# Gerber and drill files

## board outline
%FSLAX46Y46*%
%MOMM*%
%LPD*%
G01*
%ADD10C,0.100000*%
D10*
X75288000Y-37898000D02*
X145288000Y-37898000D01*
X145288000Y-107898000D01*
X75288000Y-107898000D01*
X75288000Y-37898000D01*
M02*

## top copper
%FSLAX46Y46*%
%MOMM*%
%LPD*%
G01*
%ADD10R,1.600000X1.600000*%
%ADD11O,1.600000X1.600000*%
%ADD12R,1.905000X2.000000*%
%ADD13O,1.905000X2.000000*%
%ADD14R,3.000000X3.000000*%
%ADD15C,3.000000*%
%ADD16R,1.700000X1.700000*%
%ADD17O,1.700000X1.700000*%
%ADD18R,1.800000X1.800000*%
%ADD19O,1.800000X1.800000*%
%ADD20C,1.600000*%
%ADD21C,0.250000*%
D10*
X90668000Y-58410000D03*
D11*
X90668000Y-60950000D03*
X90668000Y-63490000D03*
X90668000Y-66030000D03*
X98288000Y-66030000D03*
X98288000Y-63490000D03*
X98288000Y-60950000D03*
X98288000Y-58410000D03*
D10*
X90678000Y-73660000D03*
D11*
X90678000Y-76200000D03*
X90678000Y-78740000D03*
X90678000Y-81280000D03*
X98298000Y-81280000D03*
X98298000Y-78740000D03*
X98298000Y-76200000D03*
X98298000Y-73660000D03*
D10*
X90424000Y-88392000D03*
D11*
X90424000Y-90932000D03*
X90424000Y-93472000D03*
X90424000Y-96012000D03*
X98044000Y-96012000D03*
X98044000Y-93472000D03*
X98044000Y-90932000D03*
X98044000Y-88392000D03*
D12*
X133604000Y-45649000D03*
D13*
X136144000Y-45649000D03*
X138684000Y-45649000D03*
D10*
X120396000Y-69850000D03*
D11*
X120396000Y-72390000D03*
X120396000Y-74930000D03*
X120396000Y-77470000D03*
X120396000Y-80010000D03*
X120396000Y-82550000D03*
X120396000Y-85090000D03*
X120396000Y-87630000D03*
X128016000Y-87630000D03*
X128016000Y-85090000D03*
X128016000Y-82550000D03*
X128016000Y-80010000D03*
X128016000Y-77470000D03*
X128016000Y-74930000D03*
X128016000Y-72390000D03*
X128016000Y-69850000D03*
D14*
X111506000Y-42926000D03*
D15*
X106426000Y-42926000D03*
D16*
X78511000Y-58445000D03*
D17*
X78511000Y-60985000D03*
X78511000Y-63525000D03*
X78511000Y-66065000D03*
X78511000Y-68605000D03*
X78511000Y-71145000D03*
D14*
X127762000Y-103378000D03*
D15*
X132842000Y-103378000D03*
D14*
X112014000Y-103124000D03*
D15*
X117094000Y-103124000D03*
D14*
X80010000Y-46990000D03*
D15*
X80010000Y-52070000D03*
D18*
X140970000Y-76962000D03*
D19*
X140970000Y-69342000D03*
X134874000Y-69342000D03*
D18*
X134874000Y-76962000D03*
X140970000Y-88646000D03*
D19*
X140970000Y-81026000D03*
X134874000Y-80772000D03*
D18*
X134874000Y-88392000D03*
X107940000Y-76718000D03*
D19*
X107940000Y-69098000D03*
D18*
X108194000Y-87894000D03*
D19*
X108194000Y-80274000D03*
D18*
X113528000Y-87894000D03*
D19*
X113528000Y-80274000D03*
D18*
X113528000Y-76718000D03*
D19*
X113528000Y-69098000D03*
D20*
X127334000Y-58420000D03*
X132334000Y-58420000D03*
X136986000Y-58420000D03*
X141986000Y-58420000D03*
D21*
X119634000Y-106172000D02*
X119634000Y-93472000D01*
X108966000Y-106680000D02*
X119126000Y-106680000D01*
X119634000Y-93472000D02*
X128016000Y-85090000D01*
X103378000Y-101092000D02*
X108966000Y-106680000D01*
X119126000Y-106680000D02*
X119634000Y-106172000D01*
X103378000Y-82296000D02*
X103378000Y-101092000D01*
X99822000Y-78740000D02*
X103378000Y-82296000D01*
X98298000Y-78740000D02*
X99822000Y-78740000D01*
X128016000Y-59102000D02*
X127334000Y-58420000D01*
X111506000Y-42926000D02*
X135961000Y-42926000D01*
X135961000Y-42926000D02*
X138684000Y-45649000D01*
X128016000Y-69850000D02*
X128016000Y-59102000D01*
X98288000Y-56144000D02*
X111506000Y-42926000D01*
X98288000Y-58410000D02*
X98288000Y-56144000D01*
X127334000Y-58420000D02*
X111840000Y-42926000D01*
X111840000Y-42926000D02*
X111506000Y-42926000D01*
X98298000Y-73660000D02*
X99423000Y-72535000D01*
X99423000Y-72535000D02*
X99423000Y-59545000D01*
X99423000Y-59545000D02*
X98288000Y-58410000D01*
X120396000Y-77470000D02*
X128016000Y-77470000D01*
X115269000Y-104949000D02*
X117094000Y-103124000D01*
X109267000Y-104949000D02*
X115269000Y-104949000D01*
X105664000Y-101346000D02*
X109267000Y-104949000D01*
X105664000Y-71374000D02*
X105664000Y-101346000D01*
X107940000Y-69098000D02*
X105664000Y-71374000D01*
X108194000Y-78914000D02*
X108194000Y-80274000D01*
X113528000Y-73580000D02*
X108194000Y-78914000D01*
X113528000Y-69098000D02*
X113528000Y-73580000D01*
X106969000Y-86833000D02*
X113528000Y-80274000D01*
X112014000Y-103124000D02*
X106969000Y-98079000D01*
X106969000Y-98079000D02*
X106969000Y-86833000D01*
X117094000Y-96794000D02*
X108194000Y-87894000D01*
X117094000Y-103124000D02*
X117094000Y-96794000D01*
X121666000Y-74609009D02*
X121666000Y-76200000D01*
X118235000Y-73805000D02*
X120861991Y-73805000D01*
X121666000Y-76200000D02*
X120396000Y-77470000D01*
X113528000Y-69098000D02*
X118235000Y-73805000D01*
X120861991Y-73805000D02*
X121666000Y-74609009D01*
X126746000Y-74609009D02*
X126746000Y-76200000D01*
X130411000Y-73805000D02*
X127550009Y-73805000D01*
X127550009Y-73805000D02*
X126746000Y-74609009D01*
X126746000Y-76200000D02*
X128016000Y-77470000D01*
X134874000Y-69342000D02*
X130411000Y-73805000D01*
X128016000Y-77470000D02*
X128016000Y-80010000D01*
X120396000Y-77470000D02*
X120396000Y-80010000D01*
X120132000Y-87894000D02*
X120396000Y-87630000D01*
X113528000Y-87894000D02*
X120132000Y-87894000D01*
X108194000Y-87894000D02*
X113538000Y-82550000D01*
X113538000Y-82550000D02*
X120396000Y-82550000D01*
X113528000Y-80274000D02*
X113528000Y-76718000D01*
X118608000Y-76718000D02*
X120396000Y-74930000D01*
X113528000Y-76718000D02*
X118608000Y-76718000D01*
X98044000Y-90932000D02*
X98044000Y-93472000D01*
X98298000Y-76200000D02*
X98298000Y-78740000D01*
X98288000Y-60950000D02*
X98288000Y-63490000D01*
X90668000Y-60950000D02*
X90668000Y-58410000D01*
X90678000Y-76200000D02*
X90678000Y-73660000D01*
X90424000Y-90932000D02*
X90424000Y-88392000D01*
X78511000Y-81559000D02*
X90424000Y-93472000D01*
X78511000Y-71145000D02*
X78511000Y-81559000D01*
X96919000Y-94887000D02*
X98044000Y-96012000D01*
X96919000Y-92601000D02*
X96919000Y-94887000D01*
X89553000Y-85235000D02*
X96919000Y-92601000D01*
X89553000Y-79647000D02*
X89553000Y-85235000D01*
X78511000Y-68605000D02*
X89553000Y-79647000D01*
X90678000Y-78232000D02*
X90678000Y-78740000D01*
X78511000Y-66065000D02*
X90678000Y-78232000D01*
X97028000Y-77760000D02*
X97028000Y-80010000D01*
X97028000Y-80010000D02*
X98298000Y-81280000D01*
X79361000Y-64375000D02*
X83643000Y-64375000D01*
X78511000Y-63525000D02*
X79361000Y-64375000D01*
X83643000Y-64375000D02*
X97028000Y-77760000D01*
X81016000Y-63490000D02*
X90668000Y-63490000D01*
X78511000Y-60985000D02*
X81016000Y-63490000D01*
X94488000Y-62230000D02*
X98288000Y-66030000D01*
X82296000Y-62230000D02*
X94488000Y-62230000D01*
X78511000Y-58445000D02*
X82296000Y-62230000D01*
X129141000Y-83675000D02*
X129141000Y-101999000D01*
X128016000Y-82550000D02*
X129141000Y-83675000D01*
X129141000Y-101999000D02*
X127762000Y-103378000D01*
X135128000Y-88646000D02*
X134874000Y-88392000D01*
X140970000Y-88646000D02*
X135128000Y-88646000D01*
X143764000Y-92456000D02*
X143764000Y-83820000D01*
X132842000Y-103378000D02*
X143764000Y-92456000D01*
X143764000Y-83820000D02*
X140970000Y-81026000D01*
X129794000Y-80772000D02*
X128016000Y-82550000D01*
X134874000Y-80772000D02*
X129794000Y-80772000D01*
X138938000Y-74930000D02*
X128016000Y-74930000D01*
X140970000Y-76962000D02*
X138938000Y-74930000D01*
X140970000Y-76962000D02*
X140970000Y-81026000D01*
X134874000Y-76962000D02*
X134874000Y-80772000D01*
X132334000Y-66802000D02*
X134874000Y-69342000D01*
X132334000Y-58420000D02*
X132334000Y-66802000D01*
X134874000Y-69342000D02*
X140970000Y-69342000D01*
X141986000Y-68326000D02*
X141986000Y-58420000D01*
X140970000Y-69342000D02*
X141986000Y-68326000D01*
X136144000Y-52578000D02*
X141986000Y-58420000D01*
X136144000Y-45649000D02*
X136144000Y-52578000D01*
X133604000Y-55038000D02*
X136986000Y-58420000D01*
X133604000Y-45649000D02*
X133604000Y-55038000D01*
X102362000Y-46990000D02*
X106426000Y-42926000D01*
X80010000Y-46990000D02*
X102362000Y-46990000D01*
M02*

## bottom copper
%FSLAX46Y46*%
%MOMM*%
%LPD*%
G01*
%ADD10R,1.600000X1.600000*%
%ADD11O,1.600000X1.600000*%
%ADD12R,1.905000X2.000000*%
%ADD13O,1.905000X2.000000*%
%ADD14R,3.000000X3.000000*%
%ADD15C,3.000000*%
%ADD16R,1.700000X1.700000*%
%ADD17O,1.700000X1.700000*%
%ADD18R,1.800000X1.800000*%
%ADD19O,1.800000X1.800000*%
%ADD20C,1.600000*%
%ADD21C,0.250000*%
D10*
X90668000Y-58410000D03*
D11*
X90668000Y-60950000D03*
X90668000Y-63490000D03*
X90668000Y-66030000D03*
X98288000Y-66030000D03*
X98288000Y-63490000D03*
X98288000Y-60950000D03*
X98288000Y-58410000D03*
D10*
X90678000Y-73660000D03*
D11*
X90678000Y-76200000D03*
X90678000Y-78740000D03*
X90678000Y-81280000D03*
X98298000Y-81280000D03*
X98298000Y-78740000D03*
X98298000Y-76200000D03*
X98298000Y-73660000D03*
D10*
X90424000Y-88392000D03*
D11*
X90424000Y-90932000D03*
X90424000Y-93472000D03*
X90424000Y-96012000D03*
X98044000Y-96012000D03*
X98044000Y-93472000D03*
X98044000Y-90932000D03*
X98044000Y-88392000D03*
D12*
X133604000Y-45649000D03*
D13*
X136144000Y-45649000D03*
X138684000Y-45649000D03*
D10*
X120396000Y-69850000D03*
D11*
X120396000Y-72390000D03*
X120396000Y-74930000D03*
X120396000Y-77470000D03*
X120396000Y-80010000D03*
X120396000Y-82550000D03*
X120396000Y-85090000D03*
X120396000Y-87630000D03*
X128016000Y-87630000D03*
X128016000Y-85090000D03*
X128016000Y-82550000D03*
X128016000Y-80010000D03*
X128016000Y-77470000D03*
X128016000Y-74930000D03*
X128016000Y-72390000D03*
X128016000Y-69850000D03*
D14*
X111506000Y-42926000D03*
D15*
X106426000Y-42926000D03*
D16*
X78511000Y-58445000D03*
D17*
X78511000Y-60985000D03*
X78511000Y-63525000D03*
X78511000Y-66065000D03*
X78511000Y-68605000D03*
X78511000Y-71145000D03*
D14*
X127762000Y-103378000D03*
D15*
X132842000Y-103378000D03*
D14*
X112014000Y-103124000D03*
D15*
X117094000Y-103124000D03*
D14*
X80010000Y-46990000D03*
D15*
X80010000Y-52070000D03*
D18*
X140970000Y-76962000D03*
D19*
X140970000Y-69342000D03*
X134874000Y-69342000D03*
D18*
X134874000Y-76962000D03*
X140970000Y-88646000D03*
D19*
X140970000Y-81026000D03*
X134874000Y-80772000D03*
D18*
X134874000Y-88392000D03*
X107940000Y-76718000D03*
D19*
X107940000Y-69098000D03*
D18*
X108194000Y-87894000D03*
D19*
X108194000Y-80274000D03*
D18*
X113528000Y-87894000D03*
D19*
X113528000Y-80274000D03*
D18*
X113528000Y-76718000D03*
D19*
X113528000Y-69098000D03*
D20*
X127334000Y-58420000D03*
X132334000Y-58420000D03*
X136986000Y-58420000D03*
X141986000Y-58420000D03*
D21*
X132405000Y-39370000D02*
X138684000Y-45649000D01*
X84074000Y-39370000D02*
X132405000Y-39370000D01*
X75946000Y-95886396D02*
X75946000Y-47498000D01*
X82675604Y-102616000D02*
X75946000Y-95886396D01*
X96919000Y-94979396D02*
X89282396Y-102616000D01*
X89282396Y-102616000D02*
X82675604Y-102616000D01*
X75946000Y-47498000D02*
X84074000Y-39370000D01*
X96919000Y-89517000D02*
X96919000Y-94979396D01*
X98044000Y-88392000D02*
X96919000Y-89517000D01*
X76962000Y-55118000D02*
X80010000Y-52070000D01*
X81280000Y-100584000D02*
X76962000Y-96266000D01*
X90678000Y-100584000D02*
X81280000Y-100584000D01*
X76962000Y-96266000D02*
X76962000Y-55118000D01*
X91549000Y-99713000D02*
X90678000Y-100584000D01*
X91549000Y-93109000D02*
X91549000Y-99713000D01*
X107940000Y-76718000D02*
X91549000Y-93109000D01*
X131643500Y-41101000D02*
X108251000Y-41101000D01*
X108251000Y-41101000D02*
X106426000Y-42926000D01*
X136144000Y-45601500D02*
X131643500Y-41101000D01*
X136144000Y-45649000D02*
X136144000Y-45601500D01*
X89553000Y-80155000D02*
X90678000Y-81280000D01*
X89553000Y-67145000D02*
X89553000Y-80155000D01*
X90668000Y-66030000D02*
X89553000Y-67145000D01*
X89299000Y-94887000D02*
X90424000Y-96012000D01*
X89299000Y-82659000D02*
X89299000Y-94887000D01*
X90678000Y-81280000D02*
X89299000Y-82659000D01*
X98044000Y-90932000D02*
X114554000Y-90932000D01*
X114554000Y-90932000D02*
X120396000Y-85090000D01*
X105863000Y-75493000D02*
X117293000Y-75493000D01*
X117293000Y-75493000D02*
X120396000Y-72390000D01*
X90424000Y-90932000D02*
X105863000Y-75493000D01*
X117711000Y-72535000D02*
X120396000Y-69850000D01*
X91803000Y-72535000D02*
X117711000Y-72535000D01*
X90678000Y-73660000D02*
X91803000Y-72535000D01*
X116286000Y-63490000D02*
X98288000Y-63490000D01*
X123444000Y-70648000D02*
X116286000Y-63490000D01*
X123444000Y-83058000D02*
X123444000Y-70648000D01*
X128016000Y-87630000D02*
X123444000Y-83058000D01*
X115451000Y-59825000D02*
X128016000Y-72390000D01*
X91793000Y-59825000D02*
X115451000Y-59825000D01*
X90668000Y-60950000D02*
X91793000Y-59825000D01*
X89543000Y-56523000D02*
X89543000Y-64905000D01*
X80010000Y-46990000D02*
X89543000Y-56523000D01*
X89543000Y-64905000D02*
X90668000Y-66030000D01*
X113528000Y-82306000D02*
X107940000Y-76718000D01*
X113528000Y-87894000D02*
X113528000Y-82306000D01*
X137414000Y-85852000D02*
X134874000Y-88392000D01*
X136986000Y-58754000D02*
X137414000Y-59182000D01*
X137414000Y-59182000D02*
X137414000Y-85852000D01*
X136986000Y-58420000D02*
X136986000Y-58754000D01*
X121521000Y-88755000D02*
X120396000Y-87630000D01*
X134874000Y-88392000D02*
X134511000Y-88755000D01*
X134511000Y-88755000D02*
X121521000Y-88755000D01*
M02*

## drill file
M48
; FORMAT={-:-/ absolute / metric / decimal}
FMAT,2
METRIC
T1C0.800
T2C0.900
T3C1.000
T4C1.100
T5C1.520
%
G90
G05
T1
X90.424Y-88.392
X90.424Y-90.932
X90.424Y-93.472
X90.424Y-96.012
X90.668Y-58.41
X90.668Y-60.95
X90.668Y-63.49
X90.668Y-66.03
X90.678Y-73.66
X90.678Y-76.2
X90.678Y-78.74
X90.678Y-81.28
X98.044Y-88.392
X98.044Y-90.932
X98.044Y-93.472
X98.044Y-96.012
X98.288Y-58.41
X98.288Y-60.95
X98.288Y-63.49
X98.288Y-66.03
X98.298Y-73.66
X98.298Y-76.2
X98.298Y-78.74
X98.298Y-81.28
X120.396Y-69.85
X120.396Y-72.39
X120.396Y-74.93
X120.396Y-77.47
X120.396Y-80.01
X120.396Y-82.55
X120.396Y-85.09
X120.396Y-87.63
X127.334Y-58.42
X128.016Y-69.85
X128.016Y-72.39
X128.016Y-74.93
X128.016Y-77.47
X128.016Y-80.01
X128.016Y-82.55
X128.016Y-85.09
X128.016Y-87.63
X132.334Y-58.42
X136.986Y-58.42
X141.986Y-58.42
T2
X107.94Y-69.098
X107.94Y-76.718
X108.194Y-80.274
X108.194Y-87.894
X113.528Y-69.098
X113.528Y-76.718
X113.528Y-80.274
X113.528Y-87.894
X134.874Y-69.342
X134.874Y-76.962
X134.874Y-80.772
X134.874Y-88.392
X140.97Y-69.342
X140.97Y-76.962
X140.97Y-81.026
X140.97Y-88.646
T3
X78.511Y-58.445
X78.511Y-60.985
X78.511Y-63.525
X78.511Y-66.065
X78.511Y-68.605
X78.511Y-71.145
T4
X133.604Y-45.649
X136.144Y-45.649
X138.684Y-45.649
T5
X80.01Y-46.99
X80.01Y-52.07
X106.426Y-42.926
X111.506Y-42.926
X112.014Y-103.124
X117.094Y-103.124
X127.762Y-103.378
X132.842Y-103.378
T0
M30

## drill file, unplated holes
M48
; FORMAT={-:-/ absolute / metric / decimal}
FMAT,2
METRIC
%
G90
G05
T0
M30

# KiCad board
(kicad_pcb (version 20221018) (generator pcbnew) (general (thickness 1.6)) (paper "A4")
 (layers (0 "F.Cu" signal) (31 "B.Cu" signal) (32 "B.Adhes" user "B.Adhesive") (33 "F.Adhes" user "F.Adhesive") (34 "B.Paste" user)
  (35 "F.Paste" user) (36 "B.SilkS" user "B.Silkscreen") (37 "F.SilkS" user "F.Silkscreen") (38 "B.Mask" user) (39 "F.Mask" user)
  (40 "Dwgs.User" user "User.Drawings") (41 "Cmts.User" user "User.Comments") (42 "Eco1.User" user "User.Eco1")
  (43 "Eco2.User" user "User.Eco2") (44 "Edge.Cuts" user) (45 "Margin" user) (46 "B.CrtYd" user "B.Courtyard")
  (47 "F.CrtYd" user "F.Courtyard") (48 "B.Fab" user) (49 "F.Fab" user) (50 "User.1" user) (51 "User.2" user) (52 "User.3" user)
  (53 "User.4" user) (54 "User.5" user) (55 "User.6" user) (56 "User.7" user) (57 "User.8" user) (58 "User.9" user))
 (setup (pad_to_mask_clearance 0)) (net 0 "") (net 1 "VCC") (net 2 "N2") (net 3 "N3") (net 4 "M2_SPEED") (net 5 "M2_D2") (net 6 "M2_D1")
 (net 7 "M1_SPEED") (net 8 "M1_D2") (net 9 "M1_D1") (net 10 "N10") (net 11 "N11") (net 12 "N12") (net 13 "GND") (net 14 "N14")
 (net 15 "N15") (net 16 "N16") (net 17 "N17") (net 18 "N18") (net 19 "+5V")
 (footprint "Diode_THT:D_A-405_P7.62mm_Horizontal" (layer "F.Cu") (at 107.94 76.718 90)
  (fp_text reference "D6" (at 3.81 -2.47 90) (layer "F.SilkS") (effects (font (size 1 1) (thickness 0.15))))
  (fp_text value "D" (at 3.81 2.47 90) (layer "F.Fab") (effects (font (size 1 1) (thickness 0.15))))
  (pad "1" thru_hole rect (at 0 0 90) (size 1.8 1.8) (drill 0.9) (layers "*.Cu" "*.Mask") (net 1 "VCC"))
  (pad "2" thru_hole oval (at 7.62 0 90) (size 1.8 1.8) (drill 0.9) (layers "*.Cu" "*.Mask") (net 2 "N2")))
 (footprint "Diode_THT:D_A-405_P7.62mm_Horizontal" (layer "F.Cu") (at 140.97 88.646 90)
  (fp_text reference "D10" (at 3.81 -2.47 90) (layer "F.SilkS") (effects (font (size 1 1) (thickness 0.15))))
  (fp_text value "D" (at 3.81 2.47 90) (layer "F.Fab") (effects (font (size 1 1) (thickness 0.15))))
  (pad "1" thru_hole rect (at 0 0 90) (size 1.8 1.8) (drill 0.9) (layers "*.Cu" "*.Mask") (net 1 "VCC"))
  (pad "2" thru_hole oval (at 7.62 0 90) (size 1.8 1.8) (drill 0.9) (layers "*.Cu" "*.Mask") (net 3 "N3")))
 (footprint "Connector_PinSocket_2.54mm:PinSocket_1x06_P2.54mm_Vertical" (layer "F.Cu") (at 78.511 58.445)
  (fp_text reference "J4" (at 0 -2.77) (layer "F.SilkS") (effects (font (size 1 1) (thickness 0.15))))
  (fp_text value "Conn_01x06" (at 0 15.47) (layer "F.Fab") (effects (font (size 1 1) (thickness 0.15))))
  (pad "1" thru_hole rect (at 0 0) (size 1.7 1.7) (drill 1) (layers "*.Cu" "*.Mask") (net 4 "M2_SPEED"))
  (pad "2" thru_hole oval (at 0 2.54) (size 1.7 1.7) (drill 1) (layers "*.Cu" "*.Mask") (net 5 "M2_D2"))
  (pad "3" thru_hole oval (at 0 5.08) (size 1.7 1.7) (drill 1) (layers "*.Cu" "*.Mask") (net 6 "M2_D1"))
  (pad "4" thru_hole oval (at 0 7.62) (size 1.7 1.7) (drill 1) (layers "*.Cu" "*.Mask") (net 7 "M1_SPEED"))
  (pad "5" thru_hole oval (at 0 10.16) (size 1.7 1.7) (drill 1) (layers "*.Cu" "*.Mask") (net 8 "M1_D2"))
  (pad "6" thru_hole oval (at 0 12.7) (size 1.7 1.7) (drill 1) (layers "*.Cu" "*.Mask") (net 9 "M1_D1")))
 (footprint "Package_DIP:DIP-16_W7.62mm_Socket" (layer "F.Cu") (at 120.396 69.85)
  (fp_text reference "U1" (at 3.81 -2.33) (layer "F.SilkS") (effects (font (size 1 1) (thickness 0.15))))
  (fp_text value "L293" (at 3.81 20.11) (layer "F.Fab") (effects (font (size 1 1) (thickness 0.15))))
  (pad "1" thru_hole rect (at 0 0) (size 1.6 1.6) (drill 0.8) (layers "*.Cu" "*.Mask") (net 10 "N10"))
  (pad "2" thru_hole oval (at 0 2.54) (size 1.6 1.6) (drill 0.8) (layers "*.Cu" "*.Mask") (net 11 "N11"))
  (pad "3" thru_hole oval (at 0 5.08) (size 1.6 1.6) (drill 0.8) (layers "*.Cu" "*.Mask") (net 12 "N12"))
  (pad "4" thru_hole oval (at 0 7.62) (size 1.6 1.6) (drill 0.8) (layers "*.Cu" "*.Mask") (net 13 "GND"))
  (pad "5" thru_hole oval (at 0 10.16) (size 1.6 1.6) (drill 0.8) (layers "*.Cu" "*.Mask") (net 13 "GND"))
  (pad "6" thru_hole oval (at 0 12.7) (size 1.6 1.6) (drill 0.8) (layers "*.Cu" "*.Mask") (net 2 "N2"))
  (pad "7" thru_hole oval (at 0 15.24) (size 1.6 1.6) (drill 0.8) (layers "*.Cu" "*.Mask") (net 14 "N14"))
  (pad "8" thru_hole oval (at 0 17.78) (size 1.6 1.6) (drill 0.8) (layers "*.Cu" "*.Mask") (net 1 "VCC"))
  (pad "9" thru_hole oval (at 7.62 17.78) (size 1.6 1.6) (drill 0.8) (layers "*.Cu" "*.Mask") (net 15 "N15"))
  (pad "10" thru_hole oval (at 7.62 15.24) (size 1.6 1.6) (drill 0.8) (layers "*.Cu" "*.Mask") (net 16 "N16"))
  (pad "11" thru_hole oval (at 7.62 12.7) (size 1.6 1.6) (drill 0.8) (layers "*.Cu" "*.Mask") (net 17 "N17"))
  (pad "12" thru_hole oval (at 7.62 10.16) (size 1.6 1.6) (drill 0.8) (layers "*.Cu" "*.Mask") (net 13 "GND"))
  (pad "13" thru_hole oval (at 7.62 7.62) (size 1.6 1.6) (drill 0.8) (layers "*.Cu" "*.Mask") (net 13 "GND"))
  (pad "14" thru_hole oval (at 7.62 5.08) (size 1.6 1.6) (drill 0.8) (layers "*.Cu" "*.Mask") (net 3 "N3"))
  (pad "15" thru_hole oval (at 7.62 2.54) (size 1.6 1.6) (drill 0.8) (layers "*.Cu" "*.Mask") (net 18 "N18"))
  (pad "16" thru_hole oval (at 7.62 0) (size 1.6 1.6) (drill 0.8) (layers "*.Cu" "*.Mask") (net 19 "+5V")))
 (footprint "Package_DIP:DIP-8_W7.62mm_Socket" (layer "F.Cu") (at 90.668 58.41)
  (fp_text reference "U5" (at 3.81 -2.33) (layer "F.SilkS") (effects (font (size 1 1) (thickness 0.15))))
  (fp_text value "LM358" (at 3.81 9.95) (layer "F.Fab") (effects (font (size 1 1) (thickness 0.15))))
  (pad "1" thru_hole rect (at 0 0) (size 1.6 1.6) (drill 0.8) (layers "*.Cu" "*.Mask") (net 18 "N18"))
  (pad "2" thru_hole oval (at 0 2.54) (size 1.6 1.6) (drill 0.8) (layers "*.Cu" "*.Mask") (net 18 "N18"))
  (pad "3" thru_hole oval (at 0 5.08) (size 1.6 1.6) (drill 0.8) (layers "*.Cu" "*.Mask") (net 5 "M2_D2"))
  (pad "4" thru_hole oval (at 0 7.62) (size 1.6 1.6) (drill 0.8) (layers "*.Cu" "*.Mask") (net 13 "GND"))
  (pad "5" thru_hole oval (at 7.62 7.62) (size 1.6 1.6) (drill 0.8) (layers "*.Cu" "*.Mask") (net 4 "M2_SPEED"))
  (pad "6" thru_hole oval (at 7.62 5.08) (size 1.6 1.6) (drill 0.8) (layers "*.Cu" "*.Mask") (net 15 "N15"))
  (pad "7" thru_hole oval (at 7.62 2.54) (size 1.6 1.6) (drill 0.8) (layers "*.Cu" "*.Mask") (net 15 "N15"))
  (pad "8" thru_hole oval (at 7.62 0) (size 1.6 1.6) (drill 0.8) (layers "*.Cu" "*.Mask") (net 19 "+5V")))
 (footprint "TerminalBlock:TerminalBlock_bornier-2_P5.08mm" (layer "F.Cu") (at 127.762 103.378)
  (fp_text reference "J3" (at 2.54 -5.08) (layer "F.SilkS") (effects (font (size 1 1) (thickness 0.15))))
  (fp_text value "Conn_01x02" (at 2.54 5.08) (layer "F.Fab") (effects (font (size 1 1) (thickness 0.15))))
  (pad "1" thru_hole rect (at 0 0) (size 3 3) (drill 1.52) (layers "*.Cu" "*.Mask") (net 17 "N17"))
  (pad "2" thru_hole circle (at 5.08 0) (size 3 3) (drill 1.52) (layers "*.Cu" "*.Mask") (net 3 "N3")))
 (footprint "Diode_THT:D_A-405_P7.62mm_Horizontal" (layer "F.Cu") (at 108.194 87.894 90)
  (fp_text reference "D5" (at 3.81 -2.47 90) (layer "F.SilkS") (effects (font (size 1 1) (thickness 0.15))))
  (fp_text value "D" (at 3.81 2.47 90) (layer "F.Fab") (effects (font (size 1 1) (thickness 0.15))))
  (pad "1" thru_hole rect (at 0 0 90) (size 1.8 1.8) (drill 0.9) (layers "*.Cu" "*.Mask") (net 2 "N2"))
  (pad "2" thru_hole oval (at 7.62 0 90) (size 1.8 1.8) (drill 0.9) (layers "*.Cu" "*.Mask") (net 13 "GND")))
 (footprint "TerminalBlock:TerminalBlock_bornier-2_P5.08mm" (layer "F.Cu") (at 80.01 46.99 -90)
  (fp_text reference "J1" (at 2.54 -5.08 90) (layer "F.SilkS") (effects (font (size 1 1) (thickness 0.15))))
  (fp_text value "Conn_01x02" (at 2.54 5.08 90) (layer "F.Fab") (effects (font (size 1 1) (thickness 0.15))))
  (pad "1" thru_hole rect (at 0 0 270) (size 3 3) (drill 1.52) (layers "*.Cu" "*.Mask") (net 13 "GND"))
  (pad "2" thru_hole circle (at 5.08 0 270) (size 3 3) (drill 1.52) (layers "*.Cu" "*.Mask") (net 1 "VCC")))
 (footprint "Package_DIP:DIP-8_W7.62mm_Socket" (layer "F.Cu") (at 90.424 88.392)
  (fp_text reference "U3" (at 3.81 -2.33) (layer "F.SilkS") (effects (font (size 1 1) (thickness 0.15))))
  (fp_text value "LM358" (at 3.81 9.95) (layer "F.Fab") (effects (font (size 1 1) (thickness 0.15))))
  (pad "1" thru_hole rect (at 0 0) (size 1.6 1.6) (drill 0.8) (layers "*.Cu" "*.Mask") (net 11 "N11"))
  (pad "2" thru_hole oval (at 0 2.54) (size 1.6 1.6) (drill 0.8) (layers "*.Cu" "*.Mask") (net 11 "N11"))
  (pad "3" thru_hole oval (at 0 5.08) (size 1.6 1.6) (drill 0.8) (layers "*.Cu" "*.Mask") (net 9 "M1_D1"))
  (pad "4" thru_hole oval (at 0 7.62) (size 1.6 1.6) (drill 0.8) (layers "*.Cu" "*.Mask") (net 13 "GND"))
  (pad "5" thru_hole oval (at 7.62 7.62) (size 1.6 1.6) (drill 0.8) (layers "*.Cu" "*.Mask") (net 8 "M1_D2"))
  (pad "6" thru_hole oval (at 7.62 5.08) (size 1.6 1.6) (drill 0.8) (layers "*.Cu" "*.Mask") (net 14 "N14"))
  (pad "7" thru_hole oval (at 7.62 2.54) (size 1.6 1.6) (drill 0.8) (layers "*.Cu" "*.Mask") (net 14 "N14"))
  (pad "8" thru_hole oval (at 7.62 0) (size 1.6 1.6) (drill 0.8) (layers "*.Cu" "*.Mask") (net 19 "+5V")))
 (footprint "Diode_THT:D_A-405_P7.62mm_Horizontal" (layer "F.Cu") (at 140.97 76.962 90)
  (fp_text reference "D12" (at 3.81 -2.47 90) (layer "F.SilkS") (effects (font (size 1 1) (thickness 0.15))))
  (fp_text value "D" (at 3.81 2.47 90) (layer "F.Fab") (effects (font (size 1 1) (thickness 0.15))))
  (pad "1" thru_hole rect (at 0 0 90) (size 1.8 1.8) (drill 0.9) (layers "*.Cu" "*.Mask") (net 3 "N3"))
  (pad "2" thru_hole oval (at 7.62 0 90) (size 1.8 1.8) (drill 0.9) (layers "*.Cu" "*.Mask") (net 13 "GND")))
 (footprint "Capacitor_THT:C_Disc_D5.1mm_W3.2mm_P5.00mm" (layer "F.Cu") (at 127.334 58.42)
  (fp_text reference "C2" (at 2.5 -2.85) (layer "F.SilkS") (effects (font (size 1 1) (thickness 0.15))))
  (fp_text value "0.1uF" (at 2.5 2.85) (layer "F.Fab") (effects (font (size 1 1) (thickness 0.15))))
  (pad "1" thru_hole circle (at 0 0) (size 1.6 1.6) (drill 0.8) (layers "*.Cu" "*.Mask") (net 19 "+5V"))
  (pad "2" thru_hole circle (at 5 0) (size 1.6 1.6) (drill 0.8) (layers "*.Cu" "*.Mask") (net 13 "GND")))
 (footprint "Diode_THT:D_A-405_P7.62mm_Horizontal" (layer "F.Cu") (at 134.874 88.392 90)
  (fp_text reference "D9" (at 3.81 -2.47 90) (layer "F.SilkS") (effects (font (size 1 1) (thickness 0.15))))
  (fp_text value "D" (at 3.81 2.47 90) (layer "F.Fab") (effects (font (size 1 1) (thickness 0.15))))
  (pad "1" thru_hole rect (at 0 0 90) (size 1.8 1.8) (drill 0.9) (layers "*.Cu" "*.Mask") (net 1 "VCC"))
  (pad "2" thru_hole oval (at 7.62 0 90) (size 1.8 1.8) (drill 0.9) (layers "*.Cu" "*.Mask") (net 17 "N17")))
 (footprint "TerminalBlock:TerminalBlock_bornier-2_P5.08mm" (layer "F.Cu") (at 111.506 42.926 180)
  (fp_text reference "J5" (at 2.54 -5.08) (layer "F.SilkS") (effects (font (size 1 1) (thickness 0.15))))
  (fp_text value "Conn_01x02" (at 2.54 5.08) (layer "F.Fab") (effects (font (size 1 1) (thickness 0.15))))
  (pad "1" thru_hole rect (at 0 0 180) (size 3 3) (drill 1.52) (layers "*.Cu" "*.Mask") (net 19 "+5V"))
  (pad "2" thru_hole circle (at 5.08 0 180) (size 3 3) (drill 1.52) (layers "*.Cu" "*.Mask") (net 13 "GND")))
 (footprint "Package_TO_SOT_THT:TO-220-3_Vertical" (layer "F.Cu") (at 133.604 45.649)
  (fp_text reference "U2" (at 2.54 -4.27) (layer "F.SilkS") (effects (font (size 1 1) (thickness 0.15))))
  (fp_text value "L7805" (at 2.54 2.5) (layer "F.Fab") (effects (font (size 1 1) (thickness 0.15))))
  (pad "1" thru_hole rect (at 0 0) (size 1.905 2) (drill 1.1) (layers "*.Cu" "*.Mask") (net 1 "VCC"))
  (pad "2" thru_hole oval (at 2.54 0) (size 1.905 2) (drill 1.1) (layers "*.Cu" "*.Mask") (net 13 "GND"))
  (pad "3" thru_hole oval (at 5.08 0) (size 1.905 2) (drill 1.1) (layers "*.Cu" "*.Mask") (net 19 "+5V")))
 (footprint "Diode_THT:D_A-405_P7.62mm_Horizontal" (layer "F.Cu") (at 113.528 76.718 90)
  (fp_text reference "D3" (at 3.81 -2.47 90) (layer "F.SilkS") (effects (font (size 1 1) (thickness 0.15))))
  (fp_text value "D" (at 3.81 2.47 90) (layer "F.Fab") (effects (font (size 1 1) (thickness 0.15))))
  (pad "1" thru_hole rect (at 0 0 90) (size 1.8 1.8) (drill 0.9) (layers "*.Cu" "*.Mask") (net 12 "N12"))
  (pad "2" thru_hole oval (at 7.62 0 90) (size 1.8 1.8) (drill 0.9) (layers "*.Cu" "*.Mask") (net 13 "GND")))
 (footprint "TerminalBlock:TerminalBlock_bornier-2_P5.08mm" (layer "F.Cu") (at 112.014 103.124)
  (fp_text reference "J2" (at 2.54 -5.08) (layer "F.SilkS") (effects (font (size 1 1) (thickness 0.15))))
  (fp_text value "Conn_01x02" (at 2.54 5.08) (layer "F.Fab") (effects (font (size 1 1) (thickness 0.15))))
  (pad "1" thru_hole rect (at 0 0) (size 3 3) (drill 1.52) (layers "*.Cu" "*.Mask") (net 12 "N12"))
  (pad "2" thru_hole circle (at 5.08 0) (size 3 3) (drill 1.52) (layers "*.Cu" "*.Mask") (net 2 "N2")))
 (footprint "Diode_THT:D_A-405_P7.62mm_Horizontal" (layer "F.Cu") (at 134.874 76.962 90)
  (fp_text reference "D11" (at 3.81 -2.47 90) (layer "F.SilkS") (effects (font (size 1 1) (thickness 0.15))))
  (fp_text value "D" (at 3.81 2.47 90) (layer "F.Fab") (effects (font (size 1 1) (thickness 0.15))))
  (pad "1" thru_hole rect (at 0 0 90) (size 1.8 1.8) (drill 0.9) (layers "*.Cu" "*.Mask") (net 17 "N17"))
  (pad "2" thru_hole oval (at 7.62 0 90) (size 1.8 1.8) (drill 0.9) (layers "*.Cu" "*.Mask") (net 13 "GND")))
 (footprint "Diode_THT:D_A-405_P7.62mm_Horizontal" (layer "F.Cu") (at 113.528 87.894 90)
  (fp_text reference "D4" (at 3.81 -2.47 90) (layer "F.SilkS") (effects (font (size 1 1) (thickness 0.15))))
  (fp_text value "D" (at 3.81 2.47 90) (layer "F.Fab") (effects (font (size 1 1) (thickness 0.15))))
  (pad "1" thru_hole rect (at 0 0 90) (size 1.8 1.8) (drill 0.9) (layers "*.Cu" "*.Mask") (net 1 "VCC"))
  (pad "2" thru_hole oval (at 7.62 0 90) (size 1.8 1.8) (drill 0.9) (layers "*.Cu" "*.Mask") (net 12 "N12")))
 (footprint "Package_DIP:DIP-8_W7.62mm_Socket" (layer "F.Cu") (at 90.678 73.66)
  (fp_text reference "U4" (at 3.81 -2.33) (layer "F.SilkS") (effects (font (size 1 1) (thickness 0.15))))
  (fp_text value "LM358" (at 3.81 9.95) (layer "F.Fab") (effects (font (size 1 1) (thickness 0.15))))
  (pad "1" thru_hole rect (at 0 0) (size 1.6 1.6) (drill 0.8) (layers "*.Cu" "*.Mask") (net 10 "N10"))
  (pad "2" thru_hole oval (at 0 2.54) (size 1.6 1.6) (drill 0.8) (layers "*.Cu" "*.Mask") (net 10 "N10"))
  (pad "3" thru_hole oval (at 0 5.08) (size 1.6 1.6) (drill 0.8) (layers "*.Cu" "*.Mask") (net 7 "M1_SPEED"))
  (pad "4" thru_hole oval (at 0 7.62) (size 1.6 1.6) (drill 0.8) (layers "*.Cu" "*.Mask") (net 13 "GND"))
  (pad "5" thru_hole oval (at 7.62 7.62) (size 1.6 1.6) (drill 0.8) (layers "*.Cu" "*.Mask") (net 6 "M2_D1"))
  (pad "6" thru_hole oval (at 7.62 5.08) (size 1.6 1.6) (drill 0.8) (layers "*.Cu" "*.Mask") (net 16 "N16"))
  (pad "7" thru_hole oval (at 7.62 2.54) (size 1.6 1.6) (drill 0.8) (layers "*.Cu" "*.Mask") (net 16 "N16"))
  (pad "8" thru_hole oval (at 7.62 0) (size 1.6 1.6) (drill 0.8) (layers "*.Cu" "*.Mask") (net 19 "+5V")))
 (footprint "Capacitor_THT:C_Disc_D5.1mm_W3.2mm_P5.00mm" (layer "F.Cu") (at 136.986 58.42)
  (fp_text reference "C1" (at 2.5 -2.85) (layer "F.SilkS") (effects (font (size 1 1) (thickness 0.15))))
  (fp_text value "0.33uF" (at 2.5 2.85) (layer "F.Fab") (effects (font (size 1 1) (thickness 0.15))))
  (pad "1" thru_hole circle (at 0 0) (size 1.6 1.6) (drill 0.8) (layers "*.Cu" "*.Mask") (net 1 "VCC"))
  (pad "2" thru_hole circle (at 5 0) (size 1.6 1.6) (drill 0.8) (layers "*.Cu" "*.Mask") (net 13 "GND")))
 (gr_rect (start 75.288 37.898) (end 145.288 107.898) (stroke (width 0.1) (type default)) (fill none) (layer "Edge.Cuts"))
 (segment (start 120.132 87.894) (end 120.396 87.63) (width 0.25) (layer "F.Cu") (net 1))
 (segment (start 133.604 45.649) (end 133.604 55.038) (width 0.25) (layer "F.Cu") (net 1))
 (segment (start 113.528 87.894) (end 120.132 87.894) (width 0.25) (layer "F.Cu") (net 1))
 (segment (start 135.128 88.646) (end 134.874 88.392) (width 0.25) (layer "F.Cu") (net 1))
 (segment (start 140.97 88.646) (end 135.128 88.646) (width 0.25) (layer "F.Cu") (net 1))
 (segment (start 133.604 55.038) (end 136.986 58.42) (width 0.25) (layer "F.Cu") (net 1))
 (segment (start 90.678 100.584) (end 81.28 100.584) (width 0.25) (layer "B.Cu") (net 1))
 (segment (start 136.986 58.42) (end 136.986 58.754) (width 0.25) (layer "B.Cu") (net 1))
 (segment (start 81.28 100.584) (end 76.962 96.266) (width 0.25) (layer "B.Cu") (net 1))
 (segment (start 134.874 88.392) (end 134.511 88.755) (width 0.25) (layer "B.Cu") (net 1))
 (segment (start 136.986 58.754) (end 137.414 59.182) (width 0.25) (layer "B.Cu") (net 1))
 (segment (start 107.94 76.718) (end 91.549 93.109) (width 0.25) (layer "B.Cu") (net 1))
 (segment (start 91.549 93.109) (end 91.549 99.713) (width 0.25) (layer "B.Cu") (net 1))
 (segment (start 76.962 55.118) (end 80.01 52.07) (width 0.25) (layer "B.Cu") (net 1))
 (segment (start 113.528 82.306) (end 107.94 76.718) (width 0.25) (layer "B.Cu") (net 1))
 (segment (start 113.528 87.894) (end 113.528 82.306) (width 0.25) (layer "B.Cu") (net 1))
 (segment (start 137.414 85.852) (end 134.874 88.392) (width 0.25) (layer "B.Cu") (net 1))
 (segment (start 134.511 88.755) (end 121.521 88.755) (width 0.25) (layer "B.Cu") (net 1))
 (segment (start 121.521 88.755) (end 120.396 87.63) (width 0.25) (layer "B.Cu") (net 1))
 (segment (start 76.962 96.266) (end 76.962 55.118) (width 0.25) (layer "B.Cu") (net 1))
 (segment (start 91.549 99.713) (end 90.678 100.584) (width 0.25) (layer "B.Cu") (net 1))
 (segment (start 137.414 59.182) (end 137.414 85.852) (width 0.25) (layer "B.Cu") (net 1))
 (segment (start 132.334 58.42) (end 132.334 66.802) (width 0.25) (layer "F.Cu") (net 13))
 (segment (start 113.528 69.098) (end 118.235 73.805) (width 0.25) (layer "F.Cu") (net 13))
 (segment (start 127.550009 73.805) (end 126.746 74.609009) (width 0.25) (layer "F.Cu") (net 13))
 (segment (start 120.861991 73.805) (end 121.666 74.609009) (width 0.25) (layer "F.Cu") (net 13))
 (segment (start 132.334 66.802) (end 134.874 69.342) (width 0.25) (layer "F.Cu") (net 13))
 (segment (start 121.666 76.2) (end 120.396 77.47) (width 0.25) (layer "F.Cu") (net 13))
 (segment (start 120.396 77.47) (end 120.396 80.01) (width 0.25) (layer "F.Cu") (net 13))
 (segment (start 136.144 52.578) (end 141.986 58.42) (width 0.25) (layer "F.Cu") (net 13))
 (segment (start 128.016 77.47) (end 128.016 80.01) (width 0.25) (layer "F.Cu") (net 13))
 (segment (start 113.528 73.58) (end 108.194 78.914) (width 0.25) (layer "F.Cu") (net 13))
 (segment (start 120.396 77.47) (end 128.016 77.47) (width 0.25) (layer "F.Cu") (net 13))
 (segment (start 126.746 74.609009) (end 126.746 76.2) (width 0.25) (layer "F.Cu") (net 13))
 (segment (start 134.874 69.342) (end 140.97 69.342) (width 0.25) (layer "F.Cu") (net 13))
 (segment (start 102.362 46.99) (end 106.426 42.926) (width 0.25) (layer "F.Cu") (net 13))
 (segment (start 113.528 69.098) (end 113.528 73.58) (width 0.25) (layer "F.Cu") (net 13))
 (segment (start 130.411 73.805) (end 127.550009 73.805) (width 0.25) (layer "F.Cu") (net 13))
 (segment (start 134.874 69.342) (end 130.411 73.805) (width 0.25) (layer "F.Cu") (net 13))
 (segment (start 108.194 78.914) (end 108.194 80.274) (width 0.25) (layer "F.Cu") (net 13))
 (segment (start 136.144 45.649) (end 136.144 52.578) (width 0.25) (layer "F.Cu") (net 13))
 (segment (start 80.01 46.99) (end 102.362 46.99) (width 0.25) (layer "F.Cu") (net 13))
 (segment (start 118.235 73.805) (end 120.861991 73.805) (width 0.25) (layer "F.Cu") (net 13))
 (segment (start 141.986 68.326) (end 141.986 58.42) (width 0.25) (layer "F.Cu") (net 13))
 (segment (start 121.666 74.609009) (end 121.666 76.2) (width 0.25) (layer "F.Cu") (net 13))
 (segment (start 126.746 76.2) (end 128.016 77.47) (width 0.25) (layer "F.Cu") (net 13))
 (segment (start 140.97 69.342) (end 141.986 68.326) (width 0.25) (layer "F.Cu") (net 13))
 (segment (start 89.553 67.145) (end 89.553 80.155) (width 0.25) (layer "B.Cu") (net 13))
 (segment (start 89.299 82.659) (end 89.299 94.887) (width 0.25) (layer "B.Cu") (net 13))
 (segment (start 131.6435 41.101) (end 108.251 41.101) (width 0.25) (layer "B.Cu") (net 13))
 (segment (start 136.144 45.649) (end 136.144 45.6015) (width 0.25) (layer "B.Cu") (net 13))
 (segment (start 89.553 80.155) (end 90.678 81.28) (width 0.25) (layer "B.Cu") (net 13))
 (segment (start 80.01 46.99) (end 89.543 56.523) (width 0.25) (layer "B.Cu") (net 13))
 (segment (start 136.144 45.6015) (end 131.6435 41.101) (width 0.25) (layer "B.Cu") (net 13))
 (segment (start 90.668 66.03) (end 89.553 67.145) (width 0.25) (layer "B.Cu") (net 13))
 (segment (start 89.299 94.887) (end 90.424 96.012) (width 0.25) (layer "B.Cu") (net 13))
 (segment (start 108.251 41.101) (end 106.426 42.926) (width 0.25) (layer "B.Cu") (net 13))
 (segment (start 89.543 56.523) (end 89.543 64.905) (width 0.25) (layer "B.Cu") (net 13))
 (segment (start 90.678 81.28) (end 89.299 82.659) (width 0.25) (layer "B.Cu") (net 13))
 (segment (start 89.543 64.905) (end 90.668 66.03) (width 0.25) (layer "B.Cu") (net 13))
 (segment (start 98.288 56.144) (end 111.506 42.926) (width 0.25) (layer "F.Cu") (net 19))
 (segment (start 127.334 58.42) (end 111.84 42.926) (width 0.25) (layer "F.Cu") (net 19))
 (segment (start 111.506 42.926) (end 135.961 42.926) (width 0.25) (layer "F.Cu") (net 19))
 (segment (start 128.016 69.85) (end 128.016 59.102) (width 0.25) (layer "F.Cu") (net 19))
 (segment (start 99.423 72.535) (end 99.423 59.545) (width 0.25) (layer "F.Cu") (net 19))
 (segment (start 98.288 58.41) (end 98.288 56.144) (width 0.25) (layer "F.Cu") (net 19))
 (segment (start 98.298 73.66) (end 99.423 72.535) (width 0.25) (layer "F.Cu") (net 19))
 (segment (start 111.84 42.926) (end 111.506 42.926) (width 0.25) (layer "F.Cu") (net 19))
 (segment (start 135.961 42.926) (end 138.684 45.649) (width 0.25) (layer "F.Cu") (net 19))
 (segment (start 99.423 59.545) (end 98.288 58.41) (width 0.25) (layer "F.Cu") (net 19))
 (segment (start 128.016 59.102) (end 127.334 58.42) (width 0.25) (layer "F.Cu") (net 19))
 (segment (start 84.074 39.37) (end 132.405 39.37) (width 0.25) (layer "B.Cu") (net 19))
 (segment (start 89.282396 102.616) (end 82.675604 102.616) (width 0.25) (layer "B.Cu") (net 19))
 (segment (start 96.919 94.979396) (end 89.282396 102.616) (width 0.25) (layer "B.Cu") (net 19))
 (segment (start 82.675604 102.616) (end 75.946 95.886396) (width 0.25) (layer "B.Cu") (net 19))
 (segment (start 75.946 47.498) (end 84.074 39.37) (width 0.25) (layer "B.Cu") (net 19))
 (segment (start 75.946 95.886396) (end 75.946 47.498) (width 0.25) (layer "B.Cu") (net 19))
 (segment (start 132.405 39.37) (end 138.684 45.649) (width 0.25) (layer "B.Cu") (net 19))
 (segment (start 98.044 88.392) (end 96.919 89.517) (width 0.25) (layer "B.Cu") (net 19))
 (segment (start 96.919 89.517) (end 96.919 94.979396) (width 0.25) (layer "B.Cu") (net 19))
 (segment (start 106.969 86.833) (end 113.528 80.274) (width 0.25) (layer "F.Cu") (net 12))
 (segment (start 113.528 80.274) (end 113.528 76.718) (width 0.25) (layer "F.Cu") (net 12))
 (segment (start 118.608 76.718) (end 120.396 74.93) (width 0.25) (layer "F.Cu") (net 12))
 (segment (start 112.014 103.124) (end 106.969 98.079) (width 0.25) (layer "F.Cu") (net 12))
 (segment (start 106.969 98.079) (end 106.969 86.833) (width 0.25) (layer "F.Cu") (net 12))
 (segment (start 113.528 76.718) (end 118.608 76.718) (width 0.25) (layer "F.Cu") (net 12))
 (segment (start 105.664 101.346) (end 109.267 104.949) (width 0.25) (layer "F.Cu") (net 2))
 (segment (start 105.664 71.374) (end 105.664 101.346) (width 0.25) (layer "F.Cu") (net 2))
 (segment (start 117.094 96.794) (end 108.194 87.894) (width 0.25) (layer "F.Cu") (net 2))
 (segment (start 107.94 69.098) (end 105.664 71.374) (width 0.25) (layer "F.Cu") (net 2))
 (segment (start 109.267 104.949) (end 115.269 104.949) (width 0.25) (layer "F.Cu") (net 2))
 (segment (start 117.094 103.124) (end 117.094 96.794) (width 0.25) (layer "F.Cu") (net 2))
 (segment (start 115.269 104.949) (end 117.094 103.124) (width 0.25) (layer "F.Cu") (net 2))
 (segment (start 113.538 82.55) (end 120.396 82.55) (width 0.25) (layer "F.Cu") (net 2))
 (segment (start 108.194 87.894) (end 113.538 82.55) (width 0.25) (layer "F.Cu") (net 2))
 (segment (start 134.874 80.772) (end 129.794 80.772) (width 0.25) (layer "F.Cu") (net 17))
 (segment (start 129.794 80.772) (end 128.016 82.55) (width 0.25) (layer "F.Cu") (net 17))
 (segment (start 129.141 101.999) (end 127.762 103.378) (width 0.25) (layer "F.Cu") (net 17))
 (segment (start 129.141 83.675) (end 129.141 101.999) (width 0.25) (layer "F.Cu") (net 17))
 (segment (start 128.016 82.55) (end 129.141 83.675) (width 0.25) (layer "F.Cu") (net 17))
 (segment (start 134.874 76.962) (end 134.874 80.772) (width 0.25) (layer "F.Cu") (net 17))
 (segment (start 138.938 74.93) (end 128.016 74.93) (width 0.25) (layer "F.Cu") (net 3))
 (segment (start 143.764 83.82) (end 140.97 81.026) (width 0.25) (layer "F.Cu") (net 3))
 (segment (start 143.764 92.456) (end 143.764 83.82) (width 0.25) (layer "F.Cu") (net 3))
 (segment (start 132.842 103.378) (end 143.764 92.456) (width 0.25) (layer "F.Cu") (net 3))
 (segment (start 140.97 76.962) (end 138.938 74.93) (width 0.25) (layer "F.Cu") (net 3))
 (segment (start 140.97 76.962) (end 140.97 81.026) (width 0.25) (layer "F.Cu") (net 3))
 (segment (start 78.511 58.445) (end 82.296 62.23) (width 0.25) (layer "F.Cu") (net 4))
 (segment (start 82.296 62.23) (end 94.488 62.23) (width 0.25) (layer "F.Cu") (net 4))
 (segment (start 94.488 62.23) (end 98.288 66.03) (width 0.25) (layer "F.Cu") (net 4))
 (segment (start 78.511 60.985) (end 81.016 63.49) (width 0.25) (layer "F.Cu") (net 5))
 (segment (start 81.016 63.49) (end 90.668 63.49) (width 0.25) (layer "F.Cu") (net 5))
 (segment (start 97.028 80.01) (end 98.298 81.28) (width 0.25) (layer "F.Cu") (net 6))
 (segment (start 79.361 64.375) (end 83.643 64.375) (width 0.25) (layer "F.Cu") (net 6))
 (segment (start 78.511 63.525) (end 79.361 64.375) (width 0.25) (layer "F.Cu") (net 6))
 (segment (start 97.028 77.76) (end 97.028 80.01) (width 0.25) (layer "F.Cu") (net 6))
 (segment (start 83.643 64.375) (end 97.028 77.76) (width 0.25) (layer "F.Cu") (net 6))
 (segment (start 78.511 66.065) (end 90.678 78.232) (width 0.25) (layer "F.Cu") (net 7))
 (segment (start 90.678 78.232) (end 90.678 78.74) (width 0.25) (layer "F.Cu") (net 7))
 (segment (start 89.553 85.235) (end 96.919 92.601) (width 0.25) (layer "F.Cu") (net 8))
 (segment (start 96.919 92.601) (end 96.919 94.887) (width 0.25) (layer "F.Cu") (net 8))
 (segment (start 89.553 79.647) (end 89.553 85.235) (width 0.25) (layer "F.Cu") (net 8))
 (segment (start 78.511 68.605) (end 89.553 79.647) (width 0.25) (layer "F.Cu") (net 8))
 (segment (start 96.919 94.887) (end 98.044 96.012) (width 0.25) (layer "F.Cu") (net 8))
 (segment (start 78.511 71.145) (end 78.511 81.559) (width 0.25) (layer "F.Cu") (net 9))
 (segment (start 78.511 81.559) (end 90.424 93.472) (width 0.25) (layer "F.Cu") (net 9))
 (segment (start 90.678 76.2) (end 90.678 73.66) (width 0.25) (layer "F.Cu") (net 10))
 (segment (start 117.711 72.535) (end 120.396 69.85) (width 0.25) (layer "B.Cu") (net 10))
 (segment (start 90.678 73.66) (end 91.803 72.535) (width 0.25) (layer "B.Cu") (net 10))
 (segment (start 91.803 72.535) (end 117.711 72.535) (width 0.25) (layer "B.Cu") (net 10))
 (segment (start 90.424 90.932) (end 90.424 88.392) (width 0.25) (layer "F.Cu") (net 11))
 (segment (start 117.293 75.493) (end 120.396 72.39) (width 0.25) (layer "B.Cu") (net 11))
 (segment (start 105.863 75.493) (end 117.293 75.493) (width 0.25) (layer "B.Cu") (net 11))
 (segment (start 90.424 90.932) (end 105.863 75.493) (width 0.25) (layer "B.Cu") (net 11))
 (segment (start 98.044 90.932) (end 98.044 93.472) (width 0.25) (layer "F.Cu") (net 14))
 (segment (start 114.554 90.932) (end 120.396 85.09) (width 0.25) (layer "B.Cu") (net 14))
 (segment (start 98.044 90.932) (end 114.554 90.932) (width 0.25) (layer "B.Cu") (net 14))
 (segment (start 98.288 60.95) (end 98.288 63.49) (width 0.25) (layer "F.Cu") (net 15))
 (segment (start 116.286 63.49) (end 98.288 63.49) (width 0.25) (layer "B.Cu") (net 15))
 (segment (start 123.444 70.648) (end 116.286 63.49) (width 0.25) (layer "B.Cu") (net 15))
 (segment (start 123.444 83.058) (end 123.444 70.648) (width 0.25) (layer "B.Cu") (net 15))
 (segment (start 128.016 87.63) (end 123.444 83.058) (width 0.25) (layer "B.Cu") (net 15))
 (segment (start 98.298 76.2) (end 98.298 78.74) (width 0.25) (layer "F.Cu") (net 16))
 (segment (start 103.378 82.296) (end 103.378 101.092) (width 0.25) (layer "F.Cu") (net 16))
 (segment (start 119.126 106.68) (end 119.634 106.172) (width 0.25) (layer "F.Cu") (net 16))
 (segment (start 99.822 78.74) (end 103.378 82.296) (width 0.25) (layer "F.Cu") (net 16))
 (segment (start 98.298 78.74) (end 99.822 78.74) (width 0.25) (layer "F.Cu") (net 16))
 (segment (start 119.634 93.472) (end 128.016 85.09) (width 0.25) (layer "F.Cu") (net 16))
 (segment (start 103.378 101.092) (end 108.966 106.68) (width 0.25) (layer "F.Cu") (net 16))
 (segment (start 119.634 106.172) (end 119.634 93.472) (width 0.25) (layer "F.Cu") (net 16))
 (segment (start 108.966 106.68) (end 119.126 106.68) (width 0.25) (layer "F.Cu") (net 16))
 (segment (start 90.668 60.95) (end 90.668 58.41) (width 0.25) (layer "F.Cu") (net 18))
 (segment (start 90.668 60.95) (end 91.793 59.825) (width 0.25) (layer "B.Cu") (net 18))
 (segment (start 115.451 59.825) (end 128.016 72.39) (width 0.25) (layer "B.Cu") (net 18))
 (segment (start 91.793 59.825) (end 115.451 59.825) (width 0.25) (layer "B.Cu") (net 18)))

